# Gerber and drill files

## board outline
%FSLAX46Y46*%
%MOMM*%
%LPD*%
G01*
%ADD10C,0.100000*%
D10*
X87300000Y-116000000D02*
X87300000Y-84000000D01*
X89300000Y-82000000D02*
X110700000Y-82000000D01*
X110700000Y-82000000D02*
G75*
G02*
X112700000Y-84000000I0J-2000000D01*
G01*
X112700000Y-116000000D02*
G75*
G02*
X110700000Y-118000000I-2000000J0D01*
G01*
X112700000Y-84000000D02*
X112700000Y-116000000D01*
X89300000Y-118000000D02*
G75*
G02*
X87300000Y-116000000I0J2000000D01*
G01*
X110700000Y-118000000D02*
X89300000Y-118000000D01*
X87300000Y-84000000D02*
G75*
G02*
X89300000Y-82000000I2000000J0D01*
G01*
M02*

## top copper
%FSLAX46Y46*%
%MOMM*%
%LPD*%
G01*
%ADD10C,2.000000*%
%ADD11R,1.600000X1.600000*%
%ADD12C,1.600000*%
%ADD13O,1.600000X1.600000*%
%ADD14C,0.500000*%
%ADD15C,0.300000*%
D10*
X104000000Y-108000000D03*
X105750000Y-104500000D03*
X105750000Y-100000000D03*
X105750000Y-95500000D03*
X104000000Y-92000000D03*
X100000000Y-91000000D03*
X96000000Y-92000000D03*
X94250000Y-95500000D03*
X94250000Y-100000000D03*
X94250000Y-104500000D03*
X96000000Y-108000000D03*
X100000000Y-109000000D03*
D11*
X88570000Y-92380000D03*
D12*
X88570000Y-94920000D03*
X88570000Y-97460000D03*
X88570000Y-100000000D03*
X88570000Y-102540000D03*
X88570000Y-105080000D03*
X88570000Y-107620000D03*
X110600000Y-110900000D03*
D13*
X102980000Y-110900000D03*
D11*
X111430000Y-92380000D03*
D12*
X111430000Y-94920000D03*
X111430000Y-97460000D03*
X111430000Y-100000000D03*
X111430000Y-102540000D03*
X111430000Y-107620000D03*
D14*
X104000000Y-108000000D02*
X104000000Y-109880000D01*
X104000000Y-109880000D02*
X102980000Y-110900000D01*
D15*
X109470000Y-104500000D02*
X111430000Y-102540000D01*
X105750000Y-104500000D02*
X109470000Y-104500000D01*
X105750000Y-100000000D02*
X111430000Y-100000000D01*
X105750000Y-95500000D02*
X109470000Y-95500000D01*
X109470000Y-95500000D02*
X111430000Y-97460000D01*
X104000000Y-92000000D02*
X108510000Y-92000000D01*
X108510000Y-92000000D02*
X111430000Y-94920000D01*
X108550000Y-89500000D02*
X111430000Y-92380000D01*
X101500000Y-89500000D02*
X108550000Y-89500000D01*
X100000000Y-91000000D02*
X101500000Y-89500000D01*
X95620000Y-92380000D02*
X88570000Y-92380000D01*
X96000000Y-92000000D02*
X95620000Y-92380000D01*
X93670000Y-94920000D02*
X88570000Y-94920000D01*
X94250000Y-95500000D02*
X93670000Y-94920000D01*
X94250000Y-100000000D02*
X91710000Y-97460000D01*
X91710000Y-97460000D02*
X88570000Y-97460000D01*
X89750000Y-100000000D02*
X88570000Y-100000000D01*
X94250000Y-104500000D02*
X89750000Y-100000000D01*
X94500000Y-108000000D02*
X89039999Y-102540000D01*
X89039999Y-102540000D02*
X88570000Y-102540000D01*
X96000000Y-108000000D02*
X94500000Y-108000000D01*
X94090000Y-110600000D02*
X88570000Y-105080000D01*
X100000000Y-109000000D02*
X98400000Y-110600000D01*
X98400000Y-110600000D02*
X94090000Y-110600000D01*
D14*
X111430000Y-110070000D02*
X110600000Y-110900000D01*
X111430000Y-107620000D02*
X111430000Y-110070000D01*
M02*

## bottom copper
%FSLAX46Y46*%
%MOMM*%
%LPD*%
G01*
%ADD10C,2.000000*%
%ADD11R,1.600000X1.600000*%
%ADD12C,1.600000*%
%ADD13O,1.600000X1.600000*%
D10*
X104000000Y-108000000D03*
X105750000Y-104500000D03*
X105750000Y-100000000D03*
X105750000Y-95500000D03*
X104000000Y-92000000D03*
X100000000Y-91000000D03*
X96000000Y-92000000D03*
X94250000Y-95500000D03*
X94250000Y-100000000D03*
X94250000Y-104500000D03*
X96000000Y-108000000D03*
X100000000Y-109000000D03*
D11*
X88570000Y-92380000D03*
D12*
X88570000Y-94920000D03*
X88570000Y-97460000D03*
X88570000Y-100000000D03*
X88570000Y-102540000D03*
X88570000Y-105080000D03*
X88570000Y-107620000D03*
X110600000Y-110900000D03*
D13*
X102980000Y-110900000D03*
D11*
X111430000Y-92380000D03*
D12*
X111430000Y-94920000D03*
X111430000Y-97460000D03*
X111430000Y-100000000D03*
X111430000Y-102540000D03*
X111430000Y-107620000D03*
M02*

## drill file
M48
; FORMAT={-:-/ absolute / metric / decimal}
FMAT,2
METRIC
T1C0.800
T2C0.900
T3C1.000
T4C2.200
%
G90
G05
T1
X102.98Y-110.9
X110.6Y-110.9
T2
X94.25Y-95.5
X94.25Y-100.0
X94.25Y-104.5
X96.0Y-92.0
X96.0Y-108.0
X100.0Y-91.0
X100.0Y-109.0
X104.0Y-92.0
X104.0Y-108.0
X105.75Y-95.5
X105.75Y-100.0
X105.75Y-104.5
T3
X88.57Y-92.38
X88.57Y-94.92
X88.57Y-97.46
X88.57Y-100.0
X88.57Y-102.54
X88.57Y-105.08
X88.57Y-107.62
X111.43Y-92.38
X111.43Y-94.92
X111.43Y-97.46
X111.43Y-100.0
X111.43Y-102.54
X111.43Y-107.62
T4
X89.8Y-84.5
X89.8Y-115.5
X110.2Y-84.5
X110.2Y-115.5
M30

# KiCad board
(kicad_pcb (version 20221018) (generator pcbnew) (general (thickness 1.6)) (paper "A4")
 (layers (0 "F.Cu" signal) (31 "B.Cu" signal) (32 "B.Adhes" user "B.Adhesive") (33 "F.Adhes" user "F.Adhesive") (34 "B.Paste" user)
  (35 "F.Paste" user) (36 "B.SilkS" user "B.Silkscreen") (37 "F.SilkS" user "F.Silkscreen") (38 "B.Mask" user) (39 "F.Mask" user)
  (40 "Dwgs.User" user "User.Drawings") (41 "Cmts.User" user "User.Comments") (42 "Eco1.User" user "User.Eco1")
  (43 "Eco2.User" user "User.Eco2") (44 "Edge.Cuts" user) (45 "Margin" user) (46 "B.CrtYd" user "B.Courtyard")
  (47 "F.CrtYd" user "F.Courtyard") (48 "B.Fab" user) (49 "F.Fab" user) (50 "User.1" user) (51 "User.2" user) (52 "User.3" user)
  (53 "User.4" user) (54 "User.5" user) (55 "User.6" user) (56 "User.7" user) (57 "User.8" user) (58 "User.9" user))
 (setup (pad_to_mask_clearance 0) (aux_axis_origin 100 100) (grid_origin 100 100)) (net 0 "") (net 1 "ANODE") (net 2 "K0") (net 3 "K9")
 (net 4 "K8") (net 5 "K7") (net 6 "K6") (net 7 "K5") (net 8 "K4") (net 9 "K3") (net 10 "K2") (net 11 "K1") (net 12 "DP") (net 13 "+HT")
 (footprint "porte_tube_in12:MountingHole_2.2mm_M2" (layer "F.Cu") (at 110.2 115.5)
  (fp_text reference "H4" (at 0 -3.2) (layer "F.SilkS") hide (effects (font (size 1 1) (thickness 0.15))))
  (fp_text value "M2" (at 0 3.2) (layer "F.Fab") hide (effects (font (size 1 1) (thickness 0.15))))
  (pad "" np_thru_hole circle (at 0 0) (size 2.2 2.2) (drill 2.2) (layers "*.Cu" "*.Mask")))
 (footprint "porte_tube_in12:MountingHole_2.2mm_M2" (layer "F.Cu") (at 89.8 84.5)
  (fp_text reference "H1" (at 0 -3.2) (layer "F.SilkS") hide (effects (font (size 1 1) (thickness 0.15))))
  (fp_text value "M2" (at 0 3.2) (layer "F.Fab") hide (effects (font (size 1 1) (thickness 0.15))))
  (pad "" np_thru_hole circle (at 0 0) (size 2.2 2.2) (drill 2.2) (layers "*.Cu" "*.Mask")))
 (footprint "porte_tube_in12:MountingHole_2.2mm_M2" (layer "F.Cu") (at 110.2 84.5)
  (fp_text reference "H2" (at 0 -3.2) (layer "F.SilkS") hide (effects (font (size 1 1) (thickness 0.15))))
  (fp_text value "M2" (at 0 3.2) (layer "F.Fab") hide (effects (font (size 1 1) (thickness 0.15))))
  (pad "" np_thru_hole circle (at 0 0) (size 2.2 2.2) (drill 2.2) (layers "*.Cu" "*.Mask")))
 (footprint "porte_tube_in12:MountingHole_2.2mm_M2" (layer "F.Cu") (at 89.8 115.5)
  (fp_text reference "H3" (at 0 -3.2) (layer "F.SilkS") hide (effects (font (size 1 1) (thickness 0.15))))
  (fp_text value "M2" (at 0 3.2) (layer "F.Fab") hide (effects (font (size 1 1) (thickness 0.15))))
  (pad "" np_thru_hole circle (at 0 0) (size 2.2 2.2) (drill 2.2) (layers "*.Cu" "*.Mask")))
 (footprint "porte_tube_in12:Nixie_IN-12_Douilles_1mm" (layer "F.Cu") (at 100 100)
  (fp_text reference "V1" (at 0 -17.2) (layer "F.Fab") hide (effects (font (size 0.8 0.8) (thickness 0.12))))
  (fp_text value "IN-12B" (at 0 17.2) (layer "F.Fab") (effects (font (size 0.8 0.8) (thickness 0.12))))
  (pad "1" thru_hole circle (at 4 8) (size 2 2) (drill 0.9) (layers "*.Cu" "*.Mask") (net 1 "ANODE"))
  (pad "2" thru_hole circle (at 5.75 4.5) (size 2 2) (drill 0.9) (layers "*.Cu" "*.Mask") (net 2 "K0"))
  (pad "3" thru_hole circle (at 5.75 0) (size 2 2) (drill 0.9) (layers "*.Cu" "*.Mask") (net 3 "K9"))
  (pad "4" thru_hole circle (at 5.75 -4.5) (size 2 2) (drill 0.9) (layers "*.Cu" "*.Mask") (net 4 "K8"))
  (pad "5" thru_hole circle (at 4 -8) (size 2 2) (drill 0.9) (layers "*.Cu" "*.Mask") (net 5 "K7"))
  (pad "6" thru_hole circle (at 0 -9) (size 2 2) (drill 0.9) (layers "*.Cu" "*.Mask") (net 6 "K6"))
  (pad "7" thru_hole circle (at -4 -8) (size 2 2) (drill 0.9) (layers "*.Cu" "*.Mask") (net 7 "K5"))
  (pad "8" thru_hole circle (at -5.75 -4.5) (size 2 2) (drill 0.9) (layers "*.Cu" "*.Mask") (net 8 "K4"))
  (pad "9" thru_hole circle (at -5.75 0) (size 2 2) (drill 0.9) (layers "*.Cu" "*.Mask") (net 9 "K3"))
  (pad "10" thru_hole circle (at -5.75 4.5) (size 2 2) (drill 0.9) (layers "*.Cu" "*.Mask") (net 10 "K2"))
  (pad "11" thru_hole circle (at -4 8) (size 2 2) (drill 0.9) (layers "*.Cu" "*.Mask") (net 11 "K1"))
  (pad "12" thru_hole circle (at 0 9) (size 2 2) (drill 0.9) (layers "*.Cu" "*.Mask") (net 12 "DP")))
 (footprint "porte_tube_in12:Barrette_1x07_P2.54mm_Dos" (layer "B.Cu") (at 88.57 92.38 180)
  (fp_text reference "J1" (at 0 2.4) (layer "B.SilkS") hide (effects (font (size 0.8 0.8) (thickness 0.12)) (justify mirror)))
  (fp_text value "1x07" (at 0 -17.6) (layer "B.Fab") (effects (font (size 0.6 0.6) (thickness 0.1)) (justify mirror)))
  (pad "1" thru_hole rect (at 0 0 180) (size 1.6 1.6) (drill 1) (layers "*.Cu" "*.Mask") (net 7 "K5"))
  (pad "2" thru_hole circle (at 0 -2.54 180) (size 1.6 1.6) (drill 1) (layers "*.Cu" "*.Mask") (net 8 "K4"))
  (pad "3" thru_hole circle (at 0 -5.08 180) (size 1.6 1.6) (drill 1) (layers "*.Cu" "*.Mask") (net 9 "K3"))
  (pad "4" thru_hole circle (at 0 -7.62 180) (size 1.6 1.6) (drill 1) (layers "*.Cu" "*.Mask") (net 10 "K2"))
  (pad "5" thru_hole circle (at 0 -10.16 180) (size 1.6 1.6) (drill 1) (layers "*.Cu" "*.Mask") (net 11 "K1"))
  (pad "6" thru_hole circle (at 0 -12.7 180) (size 1.6 1.6) (drill 1) (layers "*.Cu" "*.Mask") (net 12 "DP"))
  (pad "7" thru_hole circle (at 0 -15.24 180) (size 1.6 1.6) (drill 1) (layers "*.Cu" "*.Mask")))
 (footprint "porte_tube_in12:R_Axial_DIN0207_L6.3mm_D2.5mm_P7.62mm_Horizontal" (layer "B.Cu") (at 110.6 110.9 180)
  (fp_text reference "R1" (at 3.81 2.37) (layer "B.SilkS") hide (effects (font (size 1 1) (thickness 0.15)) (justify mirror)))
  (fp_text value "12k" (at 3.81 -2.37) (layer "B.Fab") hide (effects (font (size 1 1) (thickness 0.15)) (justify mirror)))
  (pad "1" thru_hole circle (at 0 0 180) (size 1.6 1.6) (drill 0.8) (layers "*.Cu" "*.Mask") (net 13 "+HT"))
  (pad "2" thru_hole oval (at 7.62 0 180) (size 1.6 1.6) (drill 0.8) (layers "*.Cu" "*.Mask") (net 1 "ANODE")))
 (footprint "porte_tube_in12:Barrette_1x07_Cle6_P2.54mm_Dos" (layer "B.Cu") (at 111.43 92.38 180)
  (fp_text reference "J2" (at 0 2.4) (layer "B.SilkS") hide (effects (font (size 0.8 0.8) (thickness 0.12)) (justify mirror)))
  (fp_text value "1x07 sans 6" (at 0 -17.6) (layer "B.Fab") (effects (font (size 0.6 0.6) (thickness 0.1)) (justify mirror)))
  (pad "1" thru_hole rect (at 0 0 180) (size 1.6 1.6) (drill 1) (layers "*.Cu" "*.Mask") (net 6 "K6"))
  (pad "2" thru_hole circle (at 0 -2.54 180) (size 1.6 1.6) (drill 1) (layers "*.Cu" "*.Mask") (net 5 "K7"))
  (pad "3" thru_hole circle (at 0 -5.08 180) (size 1.6 1.6) (drill 1) (layers "*.Cu" "*.Mask") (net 4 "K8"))
  (pad "4" thru_hole circle (at 0 -7.62 180) (size 1.6 1.6) (drill 1) (layers "*.Cu" "*.Mask") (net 3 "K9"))
  (pad "5" thru_hole circle (at 0 -10.16 180) (size 1.6 1.6) (drill 1) (layers "*.Cu" "*.Mask") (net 2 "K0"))
  (pad "7" thru_hole circle (at 0 -15.24 180) (size 1.6 1.6) (drill 1) (layers "*.Cu" "*.Mask") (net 13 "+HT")))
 (gr_line (start 87.3 116) (end 87.3 84) (stroke (width 0.1) (type default)) (layer "Edge.Cuts"))
 (gr_line (start 89.3 82) (end 110.7 82) (stroke (width 0.1) (type default)) (layer "Edge.Cuts"))
 (gr_arc (start 110.7 82) (mid 112.114213 82.585786) (end 112.7 84) (stroke (width 0.1) (type default)) (layer "Edge.Cuts"))
 (gr_arc (start 112.7 116) (mid 112.114213 117.414213) (end 110.7 118) (stroke (width 0.1) (type default)) (layer "Edge.Cuts"))
 (gr_line (start 112.7 84) (end 112.7 116) (stroke (width 0.1) (type default)) (layer "Edge.Cuts"))
 (gr_arc (start 89.3 118) (mid 87.885786 117.414213) (end 87.3 116) (stroke (width 0.1) (type default)) (layer "Edge.Cuts"))
 (gr_line (start 110.7 118) (end 89.3 118) (stroke (width 0.1) (type default)) (layer "Edge.Cuts"))
 (gr_arc (start 87.3 84) (mid 87.885786 82.585786) (end 89.3 82) (stroke (width 0.1) (type default)) (layer "Edge.Cuts"))
 (segment (start 104 108) (end 104 109.88) (width 0.5) (layer "F.Cu") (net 1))
 (segment (start 104 109.88) (end 102.98 110.9) (width 0.5) (layer "F.Cu") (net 1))
 (segment (start 109.47 104.5) (end 111.43 102.54) (width 0.3) (layer "F.Cu") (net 2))
 (segment (start 105.75 104.5) (end 109.47 104.5) (width 0.3) (layer "F.Cu") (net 2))
 (segment (start 105.75 100) (end 111.43 100) (width 0.3) (layer "F.Cu") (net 3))
 (segment (start 105.75 95.5) (end 109.47 95.5) (width 0.3) (layer "F.Cu") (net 4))
 (segment (start 109.47 95.5) (end 111.43 97.46) (width 0.3) (layer "F.Cu") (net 4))
 (segment (start 104 92) (end 108.51 92) (width 0.3) (layer "F.Cu") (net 5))
 (segment (start 108.51 92) (end 111.43 94.92) (width 0.3) (layer "F.Cu") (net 5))
 (segment (start 108.55 89.5) (end 111.43 92.38) (width 0.3) (layer "F.Cu") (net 6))
 (segment (start 101.5 89.5) (end 108.55 89.5) (width 0.3) (layer "F.Cu") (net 6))
 (segment (start 100 91) (end 101.5 89.5) (width 0.3) (layer "F.Cu") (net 6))
 (segment (start 95.62 92.38) (end 88.57 92.38) (width 0.3) (layer "F.Cu") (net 7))
 (segment (start 96 92) (end 95.62 92.38) (width 0.3) (layer "F.Cu") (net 7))
 (segment (start 93.67 94.92) (end 88.57 94.92) (width 0.3) (layer "F.Cu") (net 8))
 (segment (start 94.25 95.5) (end 93.67 94.92) (width 0.3) (layer "F.Cu") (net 8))
 (segment (start 94.25 100) (end 91.71 97.46) (width 0.3) (layer "F.Cu") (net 9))
 (segment (start 91.71 97.46) (end 88.57 97.46) (width 0.3) (layer "F.Cu") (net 9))
 (segment (start 89.75 100) (end 88.57 100) (width 0.3) (layer "F.Cu") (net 10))
 (segment (start 94.25 104.5) (end 89.75 100) (width 0.3) (layer "F.Cu") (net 10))
 (segment (start 94.5 108) (end 89.039999 102.54) (width 0.3) (layer "F.Cu") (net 11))
 (segment (start 89.039999 102.54) (end 88.57 102.54) (width 0.3) (layer "F.Cu") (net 11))
 (segment (start 96 108) (end 94.5 108) (width 0.3) (layer "F.Cu") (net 11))
 (segment (start 94.09 110.6) (end 88.57 105.08) (width 0.3) (layer "F.Cu") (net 12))
 (segment (start 100 109) (end 98.4 110.6) (width 0.3) (layer "F.Cu") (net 12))
 (segment (start 98.4 110.6) (end 94.09 110.6) (width 0.3) (layer "F.Cu") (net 12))
 (segment (start 111.43 110.07) (end 110.6 110.9) (width 0.5) (layer "F.Cu") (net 13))
 (segment (start 111.43 107.62) (end 111.43 110.07) (width 0.5) (layer "F.Cu") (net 13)))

